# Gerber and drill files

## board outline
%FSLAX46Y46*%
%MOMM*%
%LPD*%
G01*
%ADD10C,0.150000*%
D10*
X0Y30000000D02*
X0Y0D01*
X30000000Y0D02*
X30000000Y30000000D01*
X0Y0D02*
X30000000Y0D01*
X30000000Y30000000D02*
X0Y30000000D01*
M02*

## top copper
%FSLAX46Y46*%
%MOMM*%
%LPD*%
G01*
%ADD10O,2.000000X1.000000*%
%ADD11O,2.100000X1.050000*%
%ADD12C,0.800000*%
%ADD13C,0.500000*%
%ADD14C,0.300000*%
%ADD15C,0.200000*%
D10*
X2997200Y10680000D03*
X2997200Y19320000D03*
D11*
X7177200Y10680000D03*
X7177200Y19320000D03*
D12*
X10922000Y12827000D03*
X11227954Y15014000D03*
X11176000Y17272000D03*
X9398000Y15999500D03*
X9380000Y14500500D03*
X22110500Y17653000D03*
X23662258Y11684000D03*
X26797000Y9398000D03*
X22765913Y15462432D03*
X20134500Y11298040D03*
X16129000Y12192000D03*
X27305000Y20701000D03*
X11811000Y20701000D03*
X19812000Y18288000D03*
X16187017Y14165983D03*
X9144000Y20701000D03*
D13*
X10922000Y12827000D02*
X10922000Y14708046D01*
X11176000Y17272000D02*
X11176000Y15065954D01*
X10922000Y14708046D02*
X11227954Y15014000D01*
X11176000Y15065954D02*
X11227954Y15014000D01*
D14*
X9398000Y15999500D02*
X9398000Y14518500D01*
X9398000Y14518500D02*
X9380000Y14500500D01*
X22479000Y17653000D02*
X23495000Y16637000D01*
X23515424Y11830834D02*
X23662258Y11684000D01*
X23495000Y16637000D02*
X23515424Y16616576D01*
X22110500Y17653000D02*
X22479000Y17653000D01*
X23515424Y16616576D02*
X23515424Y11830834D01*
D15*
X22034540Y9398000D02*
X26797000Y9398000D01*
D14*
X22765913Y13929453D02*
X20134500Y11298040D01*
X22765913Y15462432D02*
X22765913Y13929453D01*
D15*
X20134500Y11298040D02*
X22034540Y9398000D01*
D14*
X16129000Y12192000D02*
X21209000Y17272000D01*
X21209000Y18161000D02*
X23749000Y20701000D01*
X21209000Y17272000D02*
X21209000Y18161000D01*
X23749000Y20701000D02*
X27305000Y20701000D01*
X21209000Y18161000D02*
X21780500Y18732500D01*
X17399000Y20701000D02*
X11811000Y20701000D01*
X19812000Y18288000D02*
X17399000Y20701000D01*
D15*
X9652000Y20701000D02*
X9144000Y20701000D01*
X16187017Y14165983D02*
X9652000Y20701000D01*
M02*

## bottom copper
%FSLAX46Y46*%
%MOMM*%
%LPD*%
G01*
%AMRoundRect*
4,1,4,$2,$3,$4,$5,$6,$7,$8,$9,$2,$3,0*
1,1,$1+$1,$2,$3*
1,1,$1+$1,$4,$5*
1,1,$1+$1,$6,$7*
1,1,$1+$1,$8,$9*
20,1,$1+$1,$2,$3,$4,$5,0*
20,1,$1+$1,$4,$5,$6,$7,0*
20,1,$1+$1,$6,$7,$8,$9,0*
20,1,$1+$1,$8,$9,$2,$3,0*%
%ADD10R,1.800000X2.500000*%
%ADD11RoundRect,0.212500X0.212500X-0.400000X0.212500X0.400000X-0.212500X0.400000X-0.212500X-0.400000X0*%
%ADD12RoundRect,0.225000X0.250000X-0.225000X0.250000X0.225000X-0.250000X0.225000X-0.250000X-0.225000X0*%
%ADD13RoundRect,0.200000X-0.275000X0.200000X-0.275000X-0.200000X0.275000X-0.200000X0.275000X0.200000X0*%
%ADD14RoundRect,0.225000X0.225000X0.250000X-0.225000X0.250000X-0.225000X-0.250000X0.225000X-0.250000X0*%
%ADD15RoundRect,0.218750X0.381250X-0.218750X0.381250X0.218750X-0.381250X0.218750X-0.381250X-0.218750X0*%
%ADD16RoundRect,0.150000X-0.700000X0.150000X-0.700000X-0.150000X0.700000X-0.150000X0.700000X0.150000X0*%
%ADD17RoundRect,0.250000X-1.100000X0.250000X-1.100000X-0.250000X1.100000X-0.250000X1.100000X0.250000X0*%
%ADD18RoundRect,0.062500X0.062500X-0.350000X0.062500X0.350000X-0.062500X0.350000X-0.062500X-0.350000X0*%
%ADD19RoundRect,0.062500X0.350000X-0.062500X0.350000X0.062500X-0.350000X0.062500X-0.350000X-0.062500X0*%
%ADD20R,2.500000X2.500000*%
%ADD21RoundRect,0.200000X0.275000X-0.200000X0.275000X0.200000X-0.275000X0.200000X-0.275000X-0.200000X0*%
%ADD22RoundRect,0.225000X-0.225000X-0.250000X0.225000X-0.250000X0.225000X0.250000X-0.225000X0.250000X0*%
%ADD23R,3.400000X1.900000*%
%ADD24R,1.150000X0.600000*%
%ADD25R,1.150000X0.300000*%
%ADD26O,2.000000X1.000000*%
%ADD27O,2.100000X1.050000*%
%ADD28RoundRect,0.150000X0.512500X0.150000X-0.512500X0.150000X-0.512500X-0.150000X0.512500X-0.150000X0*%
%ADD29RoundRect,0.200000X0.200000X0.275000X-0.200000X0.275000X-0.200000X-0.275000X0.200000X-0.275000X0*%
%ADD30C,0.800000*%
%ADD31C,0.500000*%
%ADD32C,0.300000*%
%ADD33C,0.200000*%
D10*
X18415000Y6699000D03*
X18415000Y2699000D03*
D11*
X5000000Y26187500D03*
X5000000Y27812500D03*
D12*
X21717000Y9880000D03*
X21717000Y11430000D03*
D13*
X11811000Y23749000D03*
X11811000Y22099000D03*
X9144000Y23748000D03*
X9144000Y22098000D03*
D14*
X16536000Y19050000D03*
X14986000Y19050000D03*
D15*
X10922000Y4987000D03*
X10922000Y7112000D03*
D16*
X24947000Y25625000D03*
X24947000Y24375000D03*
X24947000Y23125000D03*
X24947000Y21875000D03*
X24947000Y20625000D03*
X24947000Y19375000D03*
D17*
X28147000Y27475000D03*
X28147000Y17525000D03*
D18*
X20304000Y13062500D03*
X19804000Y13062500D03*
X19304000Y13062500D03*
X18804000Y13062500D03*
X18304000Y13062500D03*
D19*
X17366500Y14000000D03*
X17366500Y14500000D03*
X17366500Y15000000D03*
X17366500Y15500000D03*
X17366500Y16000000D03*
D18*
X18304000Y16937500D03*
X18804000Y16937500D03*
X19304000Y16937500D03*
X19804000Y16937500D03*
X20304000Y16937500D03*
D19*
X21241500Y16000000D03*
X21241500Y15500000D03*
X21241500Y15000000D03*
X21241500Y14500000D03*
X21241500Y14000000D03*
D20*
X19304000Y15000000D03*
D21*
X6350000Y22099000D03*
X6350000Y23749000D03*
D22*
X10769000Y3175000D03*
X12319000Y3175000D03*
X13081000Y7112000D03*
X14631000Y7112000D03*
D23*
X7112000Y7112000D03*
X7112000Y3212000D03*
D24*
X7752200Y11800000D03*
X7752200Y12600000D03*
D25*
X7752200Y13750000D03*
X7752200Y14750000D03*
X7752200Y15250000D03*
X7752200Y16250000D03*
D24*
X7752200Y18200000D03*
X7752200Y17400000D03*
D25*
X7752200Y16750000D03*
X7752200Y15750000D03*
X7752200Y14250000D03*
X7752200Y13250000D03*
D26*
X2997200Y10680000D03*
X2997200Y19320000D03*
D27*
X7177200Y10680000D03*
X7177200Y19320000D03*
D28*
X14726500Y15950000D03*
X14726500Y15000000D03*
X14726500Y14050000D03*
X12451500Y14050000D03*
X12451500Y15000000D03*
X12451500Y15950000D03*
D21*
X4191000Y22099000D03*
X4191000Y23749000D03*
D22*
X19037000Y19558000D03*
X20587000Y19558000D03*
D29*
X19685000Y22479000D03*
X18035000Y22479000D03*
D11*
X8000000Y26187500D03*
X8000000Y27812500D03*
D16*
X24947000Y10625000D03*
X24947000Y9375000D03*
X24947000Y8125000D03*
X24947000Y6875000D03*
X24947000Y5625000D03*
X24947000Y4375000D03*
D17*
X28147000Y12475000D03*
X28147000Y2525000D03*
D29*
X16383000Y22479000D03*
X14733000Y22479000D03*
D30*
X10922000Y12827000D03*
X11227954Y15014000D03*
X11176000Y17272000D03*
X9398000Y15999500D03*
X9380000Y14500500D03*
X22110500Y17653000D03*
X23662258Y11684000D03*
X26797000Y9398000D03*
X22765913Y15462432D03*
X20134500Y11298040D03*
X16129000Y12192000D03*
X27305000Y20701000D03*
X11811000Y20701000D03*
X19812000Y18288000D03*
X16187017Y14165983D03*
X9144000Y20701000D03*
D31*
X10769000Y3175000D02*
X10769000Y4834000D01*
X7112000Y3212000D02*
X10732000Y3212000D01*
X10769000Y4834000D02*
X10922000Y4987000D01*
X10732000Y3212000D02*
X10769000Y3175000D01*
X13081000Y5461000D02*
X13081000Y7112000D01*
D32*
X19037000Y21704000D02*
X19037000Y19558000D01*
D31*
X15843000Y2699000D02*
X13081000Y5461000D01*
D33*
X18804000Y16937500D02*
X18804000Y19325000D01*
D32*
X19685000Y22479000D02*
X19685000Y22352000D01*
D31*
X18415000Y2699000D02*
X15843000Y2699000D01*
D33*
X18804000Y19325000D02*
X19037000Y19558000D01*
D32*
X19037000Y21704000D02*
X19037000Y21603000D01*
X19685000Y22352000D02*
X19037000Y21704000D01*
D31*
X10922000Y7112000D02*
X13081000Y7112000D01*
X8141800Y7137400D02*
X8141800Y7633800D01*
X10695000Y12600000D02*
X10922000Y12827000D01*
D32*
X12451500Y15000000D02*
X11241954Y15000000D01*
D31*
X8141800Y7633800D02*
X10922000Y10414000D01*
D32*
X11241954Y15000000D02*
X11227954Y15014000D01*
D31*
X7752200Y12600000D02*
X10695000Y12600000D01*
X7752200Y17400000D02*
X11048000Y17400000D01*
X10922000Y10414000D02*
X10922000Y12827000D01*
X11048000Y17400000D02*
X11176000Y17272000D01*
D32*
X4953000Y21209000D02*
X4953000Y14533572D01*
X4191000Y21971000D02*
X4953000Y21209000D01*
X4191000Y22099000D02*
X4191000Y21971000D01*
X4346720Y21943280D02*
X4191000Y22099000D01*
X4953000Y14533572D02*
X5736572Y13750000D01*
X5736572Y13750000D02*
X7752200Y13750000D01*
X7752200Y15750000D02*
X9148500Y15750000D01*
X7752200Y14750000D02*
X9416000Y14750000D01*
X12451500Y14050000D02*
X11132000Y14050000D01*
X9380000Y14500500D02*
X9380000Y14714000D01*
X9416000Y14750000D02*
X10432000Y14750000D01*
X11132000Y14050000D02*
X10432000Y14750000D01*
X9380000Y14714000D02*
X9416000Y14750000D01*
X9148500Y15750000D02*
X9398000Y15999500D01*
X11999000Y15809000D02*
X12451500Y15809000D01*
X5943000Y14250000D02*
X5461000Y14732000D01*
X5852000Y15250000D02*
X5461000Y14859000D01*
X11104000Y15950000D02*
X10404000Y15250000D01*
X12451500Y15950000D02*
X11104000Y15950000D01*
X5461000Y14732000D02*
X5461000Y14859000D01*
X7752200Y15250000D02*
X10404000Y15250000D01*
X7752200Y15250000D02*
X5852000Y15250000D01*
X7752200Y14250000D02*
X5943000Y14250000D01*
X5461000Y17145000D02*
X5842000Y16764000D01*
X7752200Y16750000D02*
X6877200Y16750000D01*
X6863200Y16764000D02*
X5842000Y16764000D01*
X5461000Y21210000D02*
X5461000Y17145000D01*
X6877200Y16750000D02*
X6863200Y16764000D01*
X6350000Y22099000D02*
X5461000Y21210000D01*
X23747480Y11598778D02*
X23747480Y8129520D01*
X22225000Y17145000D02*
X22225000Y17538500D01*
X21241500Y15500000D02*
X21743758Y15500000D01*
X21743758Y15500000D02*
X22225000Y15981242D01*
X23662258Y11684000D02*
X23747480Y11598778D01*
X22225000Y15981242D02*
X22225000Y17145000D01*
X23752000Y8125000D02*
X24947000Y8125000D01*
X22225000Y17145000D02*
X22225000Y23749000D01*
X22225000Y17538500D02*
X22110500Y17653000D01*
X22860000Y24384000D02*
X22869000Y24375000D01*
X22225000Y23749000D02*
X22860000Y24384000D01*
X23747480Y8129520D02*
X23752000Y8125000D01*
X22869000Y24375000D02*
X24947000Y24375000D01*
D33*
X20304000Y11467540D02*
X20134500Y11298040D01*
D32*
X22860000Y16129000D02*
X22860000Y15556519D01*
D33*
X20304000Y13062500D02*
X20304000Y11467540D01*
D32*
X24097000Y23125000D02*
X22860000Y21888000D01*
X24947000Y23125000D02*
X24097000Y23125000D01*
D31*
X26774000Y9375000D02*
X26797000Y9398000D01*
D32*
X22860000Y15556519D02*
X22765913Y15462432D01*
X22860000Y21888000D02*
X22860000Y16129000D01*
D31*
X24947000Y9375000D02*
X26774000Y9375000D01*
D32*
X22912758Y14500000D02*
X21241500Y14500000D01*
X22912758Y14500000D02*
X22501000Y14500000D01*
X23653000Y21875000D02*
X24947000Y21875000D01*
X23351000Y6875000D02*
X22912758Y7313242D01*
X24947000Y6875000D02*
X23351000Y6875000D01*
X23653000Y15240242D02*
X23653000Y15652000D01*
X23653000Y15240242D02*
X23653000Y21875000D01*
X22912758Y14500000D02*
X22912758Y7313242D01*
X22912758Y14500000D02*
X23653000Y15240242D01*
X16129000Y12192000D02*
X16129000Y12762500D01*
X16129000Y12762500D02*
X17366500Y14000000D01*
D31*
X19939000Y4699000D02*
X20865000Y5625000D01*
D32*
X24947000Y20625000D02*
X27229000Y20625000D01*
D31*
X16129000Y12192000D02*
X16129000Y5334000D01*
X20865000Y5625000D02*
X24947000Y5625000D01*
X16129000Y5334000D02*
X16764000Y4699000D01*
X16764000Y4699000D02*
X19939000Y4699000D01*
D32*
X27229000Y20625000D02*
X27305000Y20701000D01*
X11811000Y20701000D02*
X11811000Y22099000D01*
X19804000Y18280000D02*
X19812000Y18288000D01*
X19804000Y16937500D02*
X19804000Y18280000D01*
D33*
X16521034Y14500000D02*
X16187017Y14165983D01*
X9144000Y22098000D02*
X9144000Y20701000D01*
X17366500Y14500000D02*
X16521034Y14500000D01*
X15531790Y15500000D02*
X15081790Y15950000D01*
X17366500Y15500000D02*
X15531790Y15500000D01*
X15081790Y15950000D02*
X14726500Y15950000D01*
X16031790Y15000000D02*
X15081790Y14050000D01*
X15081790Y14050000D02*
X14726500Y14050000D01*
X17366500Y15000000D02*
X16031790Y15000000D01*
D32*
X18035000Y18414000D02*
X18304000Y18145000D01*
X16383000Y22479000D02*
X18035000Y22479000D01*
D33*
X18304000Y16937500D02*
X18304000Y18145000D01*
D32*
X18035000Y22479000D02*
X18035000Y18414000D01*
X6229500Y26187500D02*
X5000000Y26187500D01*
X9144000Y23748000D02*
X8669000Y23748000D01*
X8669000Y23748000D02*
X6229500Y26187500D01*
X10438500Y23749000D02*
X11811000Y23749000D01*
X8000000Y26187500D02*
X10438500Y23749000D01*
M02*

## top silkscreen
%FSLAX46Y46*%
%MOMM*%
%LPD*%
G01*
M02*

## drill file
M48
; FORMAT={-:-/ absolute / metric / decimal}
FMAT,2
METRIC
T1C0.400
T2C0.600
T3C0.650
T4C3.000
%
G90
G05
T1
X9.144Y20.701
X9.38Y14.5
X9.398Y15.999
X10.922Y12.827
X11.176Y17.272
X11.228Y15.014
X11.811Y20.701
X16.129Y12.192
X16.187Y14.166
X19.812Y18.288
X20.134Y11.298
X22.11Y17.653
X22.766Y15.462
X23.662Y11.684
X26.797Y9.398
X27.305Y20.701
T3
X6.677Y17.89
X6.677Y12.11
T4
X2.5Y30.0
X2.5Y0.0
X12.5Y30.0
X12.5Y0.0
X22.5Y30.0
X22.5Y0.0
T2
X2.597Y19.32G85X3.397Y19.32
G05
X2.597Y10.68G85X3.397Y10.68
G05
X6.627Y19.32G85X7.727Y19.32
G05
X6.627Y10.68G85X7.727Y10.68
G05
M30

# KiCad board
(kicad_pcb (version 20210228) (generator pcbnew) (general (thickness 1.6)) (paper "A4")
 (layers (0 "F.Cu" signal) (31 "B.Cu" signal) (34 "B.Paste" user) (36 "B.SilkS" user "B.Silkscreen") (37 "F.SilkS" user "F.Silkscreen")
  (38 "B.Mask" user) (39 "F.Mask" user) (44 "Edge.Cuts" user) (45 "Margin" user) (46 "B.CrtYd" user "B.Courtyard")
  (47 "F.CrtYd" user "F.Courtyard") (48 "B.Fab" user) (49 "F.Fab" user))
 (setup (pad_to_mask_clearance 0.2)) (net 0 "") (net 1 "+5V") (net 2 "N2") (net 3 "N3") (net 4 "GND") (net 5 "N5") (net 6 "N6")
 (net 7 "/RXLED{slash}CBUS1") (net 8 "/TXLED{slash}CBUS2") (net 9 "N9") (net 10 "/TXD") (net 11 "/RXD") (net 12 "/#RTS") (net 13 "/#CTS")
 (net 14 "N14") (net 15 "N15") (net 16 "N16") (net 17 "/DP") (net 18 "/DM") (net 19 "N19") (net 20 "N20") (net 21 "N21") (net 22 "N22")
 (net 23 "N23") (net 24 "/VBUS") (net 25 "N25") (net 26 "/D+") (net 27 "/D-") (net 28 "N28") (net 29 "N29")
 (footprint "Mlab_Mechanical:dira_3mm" (layer "F.Cu") (at 20.574 0.254)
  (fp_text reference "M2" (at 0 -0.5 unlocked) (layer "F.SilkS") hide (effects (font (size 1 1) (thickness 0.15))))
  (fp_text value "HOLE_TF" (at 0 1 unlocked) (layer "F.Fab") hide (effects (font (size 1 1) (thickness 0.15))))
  (pad "" np_thru_hole circle (at 1.926 -0.254) (size 3 3) (drill 3) (layers *.Mask)))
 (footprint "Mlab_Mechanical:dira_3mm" (layer "F.Cu") (at 3.302 -29.845)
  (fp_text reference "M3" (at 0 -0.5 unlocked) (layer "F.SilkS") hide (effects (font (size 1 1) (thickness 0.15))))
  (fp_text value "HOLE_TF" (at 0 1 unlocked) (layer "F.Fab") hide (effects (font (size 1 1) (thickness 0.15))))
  (pad "" np_thru_hole circle (at -0.802 -0.155) (size 3 3) (drill 3) (layers *.Mask)))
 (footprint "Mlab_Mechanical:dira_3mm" (layer "F.Cu") (at 15.24 -29.972)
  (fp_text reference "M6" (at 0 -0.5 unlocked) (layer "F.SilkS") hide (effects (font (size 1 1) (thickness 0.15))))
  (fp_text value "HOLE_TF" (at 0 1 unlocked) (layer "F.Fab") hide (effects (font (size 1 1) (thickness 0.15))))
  (pad "" np_thru_hole circle (at -2.74 -0.028) (size 3 3) (drill 3) (layers *.Mask)))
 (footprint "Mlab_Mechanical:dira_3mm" (layer "F.Cu") (at 24.384 -29.845)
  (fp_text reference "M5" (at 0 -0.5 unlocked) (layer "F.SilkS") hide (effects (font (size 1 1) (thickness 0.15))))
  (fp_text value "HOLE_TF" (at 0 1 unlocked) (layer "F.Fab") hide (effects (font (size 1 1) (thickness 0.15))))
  (pad "" np_thru_hole circle (at -1.884 -0.155) (size 3 3) (drill 3) (layers *.Mask)))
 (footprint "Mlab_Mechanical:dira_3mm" (layer "F.Cu") (at 11.43 0)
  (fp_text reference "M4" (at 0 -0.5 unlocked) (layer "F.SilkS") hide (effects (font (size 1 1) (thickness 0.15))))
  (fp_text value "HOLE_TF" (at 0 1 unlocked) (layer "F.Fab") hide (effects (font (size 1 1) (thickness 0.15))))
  (pad "" np_thru_hole circle (at 1.07 0) (size 3 3) (drill 3) (layers *.Mask)))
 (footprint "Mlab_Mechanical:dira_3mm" (layer "F.Cu") (at 2.921 -0.127)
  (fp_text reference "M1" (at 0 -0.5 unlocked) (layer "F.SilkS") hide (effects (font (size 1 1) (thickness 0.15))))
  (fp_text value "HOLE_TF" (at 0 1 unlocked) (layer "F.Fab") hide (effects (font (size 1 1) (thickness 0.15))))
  (pad "" np_thru_hole circle (at -0.421 0.127) (size 3 3) (drill 3) (layers *.Mask)))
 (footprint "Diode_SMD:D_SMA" (layer "B.Cu") (at 18.415 -4.699 -90)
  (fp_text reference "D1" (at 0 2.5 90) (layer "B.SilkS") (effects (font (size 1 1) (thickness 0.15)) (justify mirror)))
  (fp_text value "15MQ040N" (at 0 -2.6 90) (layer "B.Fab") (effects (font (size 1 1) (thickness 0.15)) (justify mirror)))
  (pad "1" smd rect locked (at -2 0 270) (size 2.5 1.8) (layers "B.Cu" "B.Paste" "B.Mask") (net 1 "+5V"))
  (pad "2" smd rect locked (at 2 0 270) (size 2.5 1.8) (layers "B.Cu" "B.Paste" "B.Mask") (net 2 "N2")))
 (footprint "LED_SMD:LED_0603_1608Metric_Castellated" (layer "B.Cu") (at 5 -27 90)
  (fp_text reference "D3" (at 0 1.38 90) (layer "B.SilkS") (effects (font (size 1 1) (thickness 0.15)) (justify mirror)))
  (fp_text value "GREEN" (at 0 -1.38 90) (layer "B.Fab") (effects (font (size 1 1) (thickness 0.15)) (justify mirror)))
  (pad "1" smd roundrect locked (at -0.8125 0 90) (size 1.225 0.85) (layers "B.Cu" "B.Paste" "B.Mask") (roundrect_rratio 0.25) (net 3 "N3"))
  (pad "2" smd roundrect locked (at 0.8125 0 90) (size 1.225 0.85) (layers "B.Cu" "B.Paste" "B.Mask") (roundrect_rratio 0.25) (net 1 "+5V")))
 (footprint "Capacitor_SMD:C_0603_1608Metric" (layer "B.Cu") (at 21.717 -10.655 90)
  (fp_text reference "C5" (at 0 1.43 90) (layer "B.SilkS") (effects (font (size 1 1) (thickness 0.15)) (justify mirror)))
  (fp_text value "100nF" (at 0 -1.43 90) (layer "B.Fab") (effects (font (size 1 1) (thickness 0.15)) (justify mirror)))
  (pad "1" smd roundrect locked (at -0.775 0 90) (size 0.9 0.95) (layers "B.Cu" "B.Paste" "B.Mask") (roundrect_rratio 0.25) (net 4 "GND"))
  (pad "2" smd roundrect locked (at 0.775 0 90) (size 0.9 0.95) (layers "B.Cu" "B.Paste" "B.Mask") (roundrect_rratio 0.25) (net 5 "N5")))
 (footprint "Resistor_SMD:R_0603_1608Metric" (layer "B.Cu") (at 11.811 -22.924 -90)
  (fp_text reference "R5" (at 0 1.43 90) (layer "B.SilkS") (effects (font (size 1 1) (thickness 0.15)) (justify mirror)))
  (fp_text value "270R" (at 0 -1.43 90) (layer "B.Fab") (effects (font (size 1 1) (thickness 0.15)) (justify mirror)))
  (pad "1" smd roundrect locked (at -0.825 0 270) (size 0.8 0.95) (layers "B.Cu" "B.Paste" "B.Mask") (roundrect_rratio 0.25) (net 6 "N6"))
  (pad "2" smd roundrect locked (at 0.825 0 270) (size 0.8 0.95) (layers "B.Cu" "B.Paste" "B.Mask") (roundrect_rratio 0.25)
   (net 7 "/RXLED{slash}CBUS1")))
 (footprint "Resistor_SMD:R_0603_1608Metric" (layer "B.Cu") (at 9.144 -22.923 -90)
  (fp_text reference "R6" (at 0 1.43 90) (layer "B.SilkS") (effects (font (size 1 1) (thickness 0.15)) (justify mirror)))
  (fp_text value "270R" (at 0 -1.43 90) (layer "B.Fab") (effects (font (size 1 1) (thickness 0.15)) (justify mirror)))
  (pad "1" smd roundrect locked (at -0.825 0 270) (size 0.8 0.95) (layers "B.Cu" "B.Paste" "B.Mask") (roundrect_rratio 0.25) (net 3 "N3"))
  (pad "2" smd roundrect locked (at 0.825 0 270) (size 0.8 0.95) (layers "B.Cu" "B.Paste" "B.Mask") (roundrect_rratio 0.25)
   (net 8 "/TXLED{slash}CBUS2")))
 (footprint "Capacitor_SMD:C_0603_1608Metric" (layer "B.Cu") (at 15.761 -19.05 180)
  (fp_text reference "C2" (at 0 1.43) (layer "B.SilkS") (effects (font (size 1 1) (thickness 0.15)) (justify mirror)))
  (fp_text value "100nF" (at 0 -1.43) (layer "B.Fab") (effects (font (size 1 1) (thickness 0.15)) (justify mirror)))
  (pad "1" smd roundrect locked (at -0.775 0 180) (size 0.9 0.95) (layers "B.Cu" "B.Paste" "B.Mask") (roundrect_rratio 0.25) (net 5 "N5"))
  (pad "2" smd roundrect locked (at 0.775 0 180) (size 0.9 0.95) (layers "B.Cu" "B.Paste" "B.Mask") (roundrect_rratio 0.25) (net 4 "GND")))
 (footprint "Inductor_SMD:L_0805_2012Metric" (layer "B.Cu") (at 10.922 -6.0495 90)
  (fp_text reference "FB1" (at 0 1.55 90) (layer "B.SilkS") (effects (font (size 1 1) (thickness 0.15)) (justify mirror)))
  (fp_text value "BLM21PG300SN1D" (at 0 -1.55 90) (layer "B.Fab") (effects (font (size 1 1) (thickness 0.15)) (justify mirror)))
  (pad "1" smd roundrect locked (at -1.0625 0 90) (size 0.875 1.2) (layers "B.Cu" "B.Paste" "B.Mask") (roundrect_rratio 0.25) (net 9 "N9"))
  (pad "2" smd roundrect locked (at 1.0625 0 90) (size 0.875 1.2) (layers "B.Cu" "B.Paste" "B.Mask") (roundrect_rratio 0.25) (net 2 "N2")))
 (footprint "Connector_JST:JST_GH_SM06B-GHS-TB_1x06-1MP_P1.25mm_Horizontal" (layer "B.Cu") (at 26.797 -22.5 -90)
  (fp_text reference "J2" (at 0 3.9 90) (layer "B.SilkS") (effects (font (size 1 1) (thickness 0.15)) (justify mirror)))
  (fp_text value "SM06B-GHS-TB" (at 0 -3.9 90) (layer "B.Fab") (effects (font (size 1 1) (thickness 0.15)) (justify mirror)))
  (pad "1" smd roundrect locked (at -3.125 1.85 270) (size 0.6 1.7) (layers "B.Cu" "B.Paste" "B.Mask") (roundrect_rratio 0.25) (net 1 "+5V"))
  (pad "2" smd roundrect locked (at -1.875 1.85 270) (size 0.6 1.7) (layers "B.Cu" "B.Paste" "B.Mask") (roundrect_rratio 0.25)
   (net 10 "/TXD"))
  (pad "3" smd roundrect locked (at -0.625 1.85 270) (size 0.6 1.7) (layers "B.Cu" "B.Paste" "B.Mask") (roundrect_rratio 0.25)
   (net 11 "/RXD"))
  (pad "4" smd roundrect locked (at 0.625 1.85 270) (size 0.6 1.7) (layers "B.Cu" "B.Paste" "B.Mask") (roundrect_rratio 0.25)
   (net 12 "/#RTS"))
  (pad "5" smd roundrect locked (at 1.875 1.85 270) (size 0.6 1.7) (layers "B.Cu" "B.Paste" "B.Mask") (roundrect_rratio 0.25)
   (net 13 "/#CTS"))
  (pad "6" smd roundrect locked (at 3.125 1.85 270) (size 0.6 1.7) (layers "B.Cu" "B.Paste" "B.Mask") (roundrect_rratio 0.25) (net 4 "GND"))
  (pad "MP" smd roundrect locked (at -4.975 -1.35 270) (size 1 2.7) (layers "B.Cu" "B.Paste" "B.Mask") (roundrect_rratio 0.25) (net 4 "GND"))
  (pad "MP" smd roundrect locked (at 4.975 -1.35 270) (size 1 2.7) (layers "B.Cu" "B.Paste" "B.Mask") (roundrect_rratio 0.25) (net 4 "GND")))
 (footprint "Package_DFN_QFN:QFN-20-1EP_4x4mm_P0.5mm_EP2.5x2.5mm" (layer "B.Cu") (at 19.304 -15 90)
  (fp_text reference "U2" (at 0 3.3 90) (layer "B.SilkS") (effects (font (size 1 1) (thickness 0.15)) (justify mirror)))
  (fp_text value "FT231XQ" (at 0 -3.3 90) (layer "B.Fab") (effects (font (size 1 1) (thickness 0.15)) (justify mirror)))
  (pad "" smd roundrect locked (at -0.625 0.625 90) (size 1.01 1.01) (layers "B.Paste") (roundrect_rratio 0.247525))
  (pad "" smd roundrect locked (at 0.625 0.625 90) (size 1.01 1.01) (layers "B.Paste") (roundrect_rratio 0.247525))
  (pad "" smd roundrect locked (at -0.625 -0.625 90) (size 1.01 1.01) (layers "B.Paste") (roundrect_rratio 0.247525))
  (pad "" smd roundrect locked (at 0.625 -0.625 90) (size 1.01 1.01) (layers "B.Paste") (roundrect_rratio 0.247525))
  (pad "1" smd roundrect locked (at -1.9375 1 90) (size 0.825 0.25) (layers "B.Cu" "B.Paste" "B.Mask") (roundrect_rratio 0.25)
   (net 11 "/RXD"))
  (pad "2" smd roundrect locked (at -1.9375 0.5 90) (size 0.825 0.25) (layers "B.Cu" "B.Paste" "B.Mask") (roundrect_rratio 0.25)
   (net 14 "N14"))
  (pad "3" smd roundrect locked (at -1.9375 0 90) (size 0.825 0.25) (layers "B.Cu" "B.Paste" "B.Mask") (roundrect_rratio 0.25) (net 4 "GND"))
  (pad "4" smd roundrect locked (at -1.9375 -0.5 90) (size 0.825 0.25) (layers "B.Cu" "B.Paste" "B.Mask") (roundrect_rratio 0.25)
   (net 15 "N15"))
  (pad "5" smd roundrect locked (at -1.9375 -1 90) (size 0.825 0.25) (layers "B.Cu" "B.Paste" "B.Mask") (roundrect_rratio 0.25)
   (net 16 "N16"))
  (pad "6" smd roundrect locked (at -1 -1.9375 90) (size 0.25 0.825) (layers "B.Cu" "B.Paste" "B.Mask") (roundrect_rratio 0.25)
   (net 13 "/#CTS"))
  (pad "7" smd roundrect locked (at -0.5 -1.9375 90) (size 0.25 0.825) (layers "B.Cu" "B.Paste" "B.Mask") (roundrect_rratio 0.25)
   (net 8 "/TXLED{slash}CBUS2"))
  (pad "8" smd roundrect locked (at 0 -1.9375 90) (size 0.25 0.825) (layers "B.Cu" "B.Paste" "B.Mask") (roundrect_rratio 0.25)
   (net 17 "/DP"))
  (pad "9" smd roundrect locked (at 0.5 -1.9375 90) (size 0.25 0.825) (layers "B.Cu" "B.Paste" "B.Mask") (roundrect_rratio 0.25)
   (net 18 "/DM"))
  (pad "10" smd roundrect locked (at 1 -1.9375 90) (size 0.25 0.825) (layers "B.Cu" "B.Paste" "B.Mask") (roundrect_rratio 0.25) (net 5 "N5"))
  (pad "11" smd roundrect locked (at 1.9375 -1 90) (size 0.825 0.25) (layers "B.Cu" "B.Paste" "B.Mask") (roundrect_rratio 0.25)
   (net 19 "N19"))
  (pad "12" smd roundrect locked (at 1.9375 -0.5 90) (size 0.825 0.25) (layers "B.Cu" "B.Paste" "B.Mask") (roundrect_rratio 0.25)
   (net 2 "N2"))
  (pad "13" smd roundrect locked (at 1.9375 0 90) (size 0.825 0.25) (layers "B.Cu" "B.Paste" "B.Mask") (roundrect_rratio 0.25) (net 4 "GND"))
  (pad "14" smd roundrect locked (at 1.9375 0.5 90) (size 0.825 0.25) (layers "B.Cu" "B.Paste" "B.Mask") (roundrect_rratio 0.25)
   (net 7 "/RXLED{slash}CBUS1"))
  (pad "15" smd roundrect locked (at 1.9375 1 90) (size 0.825 0.25) (layers "B.Cu" "B.Paste" "B.Mask") (roundrect_rratio 0.25)
   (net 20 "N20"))
  (pad "16" smd roundrect locked (at 1 1.9375 90) (size 0.25 0.825) (layers "B.Cu" "B.Paste" "B.Mask") (roundrect_rratio 0.25)
   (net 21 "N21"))
  (pad "17" smd roundrect locked (at 0.5 1.9375 90) (size 0.25 0.825) (layers "B.Cu" "B.Paste" "B.Mask") (roundrect_rratio 0.25)
   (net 10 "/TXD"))
  (pad "18" smd roundrect locked (at 0 1.9375 90) (size 0.25 0.825) (layers "B.Cu" "B.Paste" "B.Mask") (roundrect_rratio 0.25)
   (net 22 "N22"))
  (pad "19" smd roundrect locked (at -0.5 1.9375 90) (size 0.25 0.825) (layers "B.Cu" "B.Paste" "B.Mask") (roundrect_rratio 0.25)
   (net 12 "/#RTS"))
  (pad "20" smd roundrect locked (at -1 1.9375 90) (size 0.25 0.825) (layers "B.Cu" "B.Paste" "B.Mask") (roundrect_rratio 0.25) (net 5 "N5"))
  (pad "21" smd rect locked (at 0 0 90) (size 2.5 2.5) (layers "B.Cu" "B.Mask") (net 4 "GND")))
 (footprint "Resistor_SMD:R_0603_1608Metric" (layer "B.Cu") (at 6.35 -22.924 90)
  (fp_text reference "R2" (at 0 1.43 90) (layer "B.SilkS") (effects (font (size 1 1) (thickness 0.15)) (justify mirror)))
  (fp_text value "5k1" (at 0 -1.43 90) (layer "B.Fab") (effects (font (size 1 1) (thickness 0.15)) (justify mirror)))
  (pad "1" smd roundrect locked (at -0.825 0 90) (size 0.8 0.95) (layers "B.Cu" "B.Paste" "B.Mask") (roundrect_rratio 0.25) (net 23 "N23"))
  (pad "2" smd roundrect locked (at 0.825 0 90) (size 0.8 0.95) (layers "B.Cu" "B.Paste" "B.Mask") (roundrect_rratio 0.25) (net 4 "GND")))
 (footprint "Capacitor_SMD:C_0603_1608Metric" (layer "B.Cu") (at 11.544 -3.175)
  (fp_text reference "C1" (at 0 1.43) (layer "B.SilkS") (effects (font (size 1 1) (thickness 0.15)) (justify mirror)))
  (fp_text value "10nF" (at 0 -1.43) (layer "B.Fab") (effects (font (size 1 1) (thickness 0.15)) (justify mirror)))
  (pad "1" smd roundrect locked (at -0.775 0) (size 0.9 0.95) (layers "B.Cu" "B.Paste" "B.Mask") (roundrect_rratio 0.25) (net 9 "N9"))
  (pad "2" smd roundrect locked (at 0.775 0) (size 0.9 0.95) (layers "B.Cu" "B.Paste" "B.Mask") (roundrect_rratio 0.25) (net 4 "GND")))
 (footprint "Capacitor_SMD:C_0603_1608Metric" (layer "B.Cu") (at 13.856 -7.112)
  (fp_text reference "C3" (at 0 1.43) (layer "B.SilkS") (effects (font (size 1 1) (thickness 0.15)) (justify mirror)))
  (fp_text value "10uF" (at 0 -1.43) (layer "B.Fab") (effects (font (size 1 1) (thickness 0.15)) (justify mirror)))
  (pad "1" smd roundrect locked (at -0.775 0) (size 0.9 0.95) (layers "B.Cu" "B.Paste" "B.Mask") (roundrect_rratio 0.25) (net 2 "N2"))
  (pad "2" smd roundrect locked (at 0.775 0) (size 0.9 0.95) (layers "B.Cu" "B.Paste" "B.Mask") (roundrect_rratio 0.25) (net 4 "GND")))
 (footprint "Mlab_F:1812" (layer "B.Cu") (at 7.112 -5.162 -90)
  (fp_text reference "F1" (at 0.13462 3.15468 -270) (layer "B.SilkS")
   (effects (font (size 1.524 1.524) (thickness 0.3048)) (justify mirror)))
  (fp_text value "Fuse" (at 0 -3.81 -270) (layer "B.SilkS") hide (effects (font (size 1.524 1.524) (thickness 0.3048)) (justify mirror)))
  (pad "1" smd rect locked (at -1.95 0 270) (size 1.9 3.4) (layers "B.Cu" "B.Paste" "B.Mask") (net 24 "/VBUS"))
  (pad "2" smd rect locked (at 1.95 0 270) (size 1.9 3.4) (layers "B.Cu" "B.Paste" "B.Mask") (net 9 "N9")))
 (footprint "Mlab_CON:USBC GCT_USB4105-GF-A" (layer "B.Cu") (at 2.9972 -15 90)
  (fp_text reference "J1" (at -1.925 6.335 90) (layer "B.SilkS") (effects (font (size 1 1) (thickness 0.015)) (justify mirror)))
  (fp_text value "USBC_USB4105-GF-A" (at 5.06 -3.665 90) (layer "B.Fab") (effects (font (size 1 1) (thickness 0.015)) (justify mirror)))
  (pad "A1/B12" smd rect locked (at -3.2 4.755 90) (size 0.6 1.15) (layers "B.Cu" "B.Paste" "B.Mask") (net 4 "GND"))
  (pad "A4/B9" smd rect locked (at -2.4 4.755 90) (size 0.6 1.15) (layers "B.Cu" "B.Paste" "B.Mask") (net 24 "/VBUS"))
  (pad "A5" smd rect locked (at -1.25 4.755 90) (size 0.3 1.15) (layers "B.Cu" "B.Paste" "B.Mask") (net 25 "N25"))
  (pad "A6" smd rect locked (at -0.25 4.755 90) (size 0.3 1.15) (layers "B.Cu" "B.Paste" "B.Mask") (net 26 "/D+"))
  (pad "A7" smd rect locked (at 0.25 4.755 90) (size 0.3 1.15) (layers "B.Cu" "B.Paste" "B.Mask") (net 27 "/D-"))
  (pad "A8" smd rect locked (at 1.25 4.755 90) (size 0.3 1.15) (layers "B.Cu" "B.Paste" "B.Mask") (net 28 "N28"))
  (pad "B1/A12" smd rect locked (at 3.2 4.755 90) (size 0.6 1.15) (layers "B.Cu" "B.Paste" "B.Mask") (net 4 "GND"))
  (pad "B4/A9" smd rect locked (at 2.4 4.755 90) (size 0.6 1.15) (layers "B.Cu" "B.Paste" "B.Mask") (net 24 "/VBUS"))
  (pad "B5" smd rect locked (at 1.75 4.755 90) (size 0.3 1.15) (layers "B.Cu" "B.Paste" "B.Mask") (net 23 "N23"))
  (pad "B6" smd rect locked (at 0.75 4.755 90) (size 0.3 1.15) (layers "B.Cu" "B.Paste" "B.Mask") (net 26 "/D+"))
  (pad "B7" smd rect locked (at -0.75 4.755 90) (size 0.3 1.15) (layers "B.Cu" "B.Paste" "B.Mask") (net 27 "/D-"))
  (pad "B8" smd rect locked (at -1.75 4.755 90) (size 0.3 1.15) (layers "B.Cu" "B.Paste" "B.Mask") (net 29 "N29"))
  (pad "G1" thru_hole oval locked (at -4.32 0 90) (size 1 2) (drill oval 0.6 1.4) (layers *.Cu *.Mask) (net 4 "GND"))
  (pad "G2" thru_hole oval locked (at 4.32 0 90) (size 1 2) (drill oval 0.6 1.4) (layers *.Cu *.Mask) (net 4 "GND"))
  (pad "G3" thru_hole oval locked (at -4.32 4.18 90) (size 1.05 2.1) (drill oval 0.6 1.7) (layers *.Cu *.Mask) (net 4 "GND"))
  (pad "G4" thru_hole oval locked (at 4.32 4.18 90) (size 1.05 2.1) (drill oval 0.6 1.7) (layers *.Cu *.Mask) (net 4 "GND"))
  (pad "None" np_thru_hole circle locked (at 2.89 3.68 90) (size 0.65 0.65) (drill 0.65) (layers *.Cu *.Mask))
  (pad "None" np_thru_hole circle locked (at -2.89 3.68 90) (size 0.65 0.65) (drill 0.65) (layers *.Cu *.Mask)))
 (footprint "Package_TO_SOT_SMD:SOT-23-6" (layer "B.Cu") (at 13.589 -15 180)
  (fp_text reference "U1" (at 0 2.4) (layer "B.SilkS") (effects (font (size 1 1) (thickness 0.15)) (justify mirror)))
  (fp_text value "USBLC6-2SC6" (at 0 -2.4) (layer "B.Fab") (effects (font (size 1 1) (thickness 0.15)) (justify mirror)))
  (pad "1" smd roundrect locked (at -1.1375 0.95 180) (size 1.325 0.6) (layers "B.Cu" "B.Paste" "B.Mask") (roundrect_rratio 0.25)
   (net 18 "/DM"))
  (pad "2" smd roundrect locked (at -1.1375 0 180) (size 1.325 0.6) (layers "B.Cu" "B.Paste" "B.Mask") (roundrect_rratio 0.25) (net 4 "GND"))
  (pad "3" smd roundrect locked (at -1.1375 -0.95 180) (size 1.325 0.6) (layers "B.Cu" "B.Paste" "B.Mask") (roundrect_rratio 0.25)
   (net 17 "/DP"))
  (pad "4" smd roundrect locked (at 1.1375 -0.95 180) (size 1.325 0.6) (layers "B.Cu" "B.Paste" "B.Mask") (roundrect_rratio 0.25)
   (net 26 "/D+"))
  (pad "5" smd roundrect locked (at 1.1375 0 180) (size 1.325 0.6) (layers "B.Cu" "B.Paste" "B.Mask") (roundrect_rratio 0.25)
   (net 24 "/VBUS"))
  (pad "6" smd roundrect locked (at 1.1375 0.95 180) (size 1.325 0.6) (layers "B.Cu" "B.Paste" "B.Mask") (roundrect_rratio 0.25)
   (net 27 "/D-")))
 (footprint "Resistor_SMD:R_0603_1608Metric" (layer "B.Cu") (at 4.191 -22.924 90)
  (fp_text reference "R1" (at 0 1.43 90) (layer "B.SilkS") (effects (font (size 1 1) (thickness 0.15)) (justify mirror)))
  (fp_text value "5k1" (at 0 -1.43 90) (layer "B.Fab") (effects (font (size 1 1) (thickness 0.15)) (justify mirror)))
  (pad "1" smd roundrect locked (at -0.825 0 90) (size 0.8 0.95) (layers "B.Cu" "B.Paste" "B.Mask") (roundrect_rratio 0.25) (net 25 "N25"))
  (pad "2" smd roundrect locked (at 0.825 0 90) (size 0.8 0.95) (layers "B.Cu" "B.Paste" "B.Mask") (roundrect_rratio 0.25) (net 4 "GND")))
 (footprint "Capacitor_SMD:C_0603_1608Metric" (layer "B.Cu") (at 19.812 -19.558)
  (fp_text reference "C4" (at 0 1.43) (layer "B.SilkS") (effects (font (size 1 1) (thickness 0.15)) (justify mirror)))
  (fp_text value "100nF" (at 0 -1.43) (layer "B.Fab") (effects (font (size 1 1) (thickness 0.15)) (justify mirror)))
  (pad "1" smd roundrect locked (at -0.775 0) (size 0.9 0.95) (layers "B.Cu" "B.Paste" "B.Mask") (roundrect_rratio 0.25) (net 2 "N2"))
  (pad "2" smd roundrect locked (at 0.775 0) (size 0.9 0.95) (layers "B.Cu" "B.Paste" "B.Mask") (roundrect_rratio 0.25) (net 4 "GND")))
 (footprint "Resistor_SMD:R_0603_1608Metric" (layer "B.Cu") (at 18.86 -22.479 180)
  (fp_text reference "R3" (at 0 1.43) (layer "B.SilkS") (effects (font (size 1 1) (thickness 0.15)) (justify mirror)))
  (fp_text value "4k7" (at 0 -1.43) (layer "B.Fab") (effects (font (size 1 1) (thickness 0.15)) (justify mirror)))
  (pad "1" smd roundrect locked (at -0.825 0 180) (size 0.8 0.95) (layers "B.Cu" "B.Paste" "B.Mask") (roundrect_rratio 0.25) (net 2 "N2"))
  (pad "2" smd roundrect locked (at 0.825 0 180) (size 0.8 0.95) (layers "B.Cu" "B.Paste" "B.Mask") (roundrect_rratio 0.25) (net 19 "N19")))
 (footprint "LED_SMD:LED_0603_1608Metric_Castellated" (layer "B.Cu") (at 8 -27 90)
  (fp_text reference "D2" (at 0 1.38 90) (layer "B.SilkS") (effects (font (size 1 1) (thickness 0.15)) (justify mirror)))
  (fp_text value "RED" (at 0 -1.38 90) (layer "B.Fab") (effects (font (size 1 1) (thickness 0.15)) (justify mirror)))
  (pad "1" smd roundrect locked (at -0.8125 0 90) (size 1.225 0.85) (layers "B.Cu" "B.Paste" "B.Mask") (roundrect_rratio 0.25) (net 6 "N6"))
  (pad "2" smd roundrect locked (at 0.8125 0 90) (size 1.225 0.85) (layers "B.Cu" "B.Paste" "B.Mask") (roundrect_rratio 0.25) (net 1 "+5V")))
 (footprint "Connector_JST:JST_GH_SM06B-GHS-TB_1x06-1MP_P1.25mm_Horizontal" (layer "B.Cu") (at 26.797 -7.5 -90)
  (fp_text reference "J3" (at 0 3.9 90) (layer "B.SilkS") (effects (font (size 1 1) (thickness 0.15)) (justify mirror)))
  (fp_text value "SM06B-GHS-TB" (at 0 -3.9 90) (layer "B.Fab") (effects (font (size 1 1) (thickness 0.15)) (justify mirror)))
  (pad "1" smd roundrect locked (at -3.125 1.85 270) (size 0.6 1.7) (layers "B.Cu" "B.Paste" "B.Mask") (roundrect_rratio 0.25) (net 1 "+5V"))
  (pad "2" smd roundrect locked (at -1.875 1.85 270) (size 0.6 1.7) (layers "B.Cu" "B.Paste" "B.Mask") (roundrect_rratio 0.25)
   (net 11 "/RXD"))
  (pad "3" smd roundrect locked (at -0.625 1.85 270) (size 0.6 1.7) (layers "B.Cu" "B.Paste" "B.Mask") (roundrect_rratio 0.25)
   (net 10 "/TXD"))
  (pad "4" smd roundrect locked (at 0.625 1.85 270) (size 0.6 1.7) (layers "B.Cu" "B.Paste" "B.Mask") (roundrect_rratio 0.25)
   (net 12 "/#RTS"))
  (pad "5" smd roundrect locked (at 1.875 1.85 270) (size 0.6 1.7) (layers "B.Cu" "B.Paste" "B.Mask") (roundrect_rratio 0.25)
   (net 13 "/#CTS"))
  (pad "6" smd roundrect locked (at 3.125 1.85 270) (size 0.6 1.7) (layers "B.Cu" "B.Paste" "B.Mask") (roundrect_rratio 0.25) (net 4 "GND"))
  (pad "MP" smd roundrect locked (at -4.975 -1.35 270) (size 1 2.7) (layers "B.Cu" "B.Paste" "B.Mask") (roundrect_rratio 0.25) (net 4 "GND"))
  (pad "MP" smd roundrect locked (at 4.975 -1.35 270) (size 1 2.7) (layers "B.Cu" "B.Paste" "B.Mask") (roundrect_rratio 0.25) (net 4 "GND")))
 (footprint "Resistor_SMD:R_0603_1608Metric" (layer "B.Cu") (at 15.558 -22.479 180)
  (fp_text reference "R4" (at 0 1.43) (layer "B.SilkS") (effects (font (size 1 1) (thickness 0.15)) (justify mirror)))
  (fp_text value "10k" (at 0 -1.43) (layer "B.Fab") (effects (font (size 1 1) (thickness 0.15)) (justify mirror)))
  (pad "1" smd roundrect locked (at -0.825 0 180) (size 0.8 0.95) (layers "B.Cu" "B.Paste" "B.Mask") (roundrect_rratio 0.25) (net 19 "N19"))
  (pad "2" smd roundrect locked (at 0.825 0 180) (size 0.8 0.95) (layers "B.Cu" "B.Paste" "B.Mask") (roundrect_rratio 0.25) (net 4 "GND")))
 (gr_line (start 0 -30) (end 0 0) (layer "Edge.Cuts") (width 0.15))
 (gr_line (start 30 0) (end 30 -30) (layer "Edge.Cuts") (width 0.15))
 (gr_line (start 0 0) (end 30 0) (layer "Edge.Cuts") (width 0.15))
 (gr_line (start 30 -30) (end 0 -30) (layer "Edge.Cuts") (width 0.15))
 (segment (start 10.769 -3.175) (end 10.769 -4.834) (width 0.5) (layer "B.Cu") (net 9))
 (segment (start 7.112 -3.212) (end 10.732 -3.212) (width 0.5) (layer "B.Cu") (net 9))
 (segment (start 10.769 -4.834) (end 10.922 -4.987) (width 0.5) (layer "B.Cu") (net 9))
 (segment (start 10.732 -3.212) (end 10.769 -3.175) (width 0.5) (layer "B.Cu") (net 9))
 (segment (start 13.081 -5.461) (end 13.081 -7.112) (width 0.5) (layer "B.Cu") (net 2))
 (segment (start 19.037 -21.704) (end 19.037 -19.558) (width 0.3) (layer "B.Cu") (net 2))
 (segment (start 15.843 -2.699) (end 13.081 -5.461) (width 0.5) (layer "B.Cu") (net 2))
 (segment (start 18.804 -16.9375) (end 18.804 -19.325) (width 0.2) (layer "B.Cu") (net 2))
 (segment (start 19.685 -22.479) (end 19.685 -22.352) (width 0.3) (layer "B.Cu") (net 2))
 (segment (start 18.415 -2.699) (end 15.843 -2.699) (width 0.5) (layer "B.Cu") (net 2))
 (segment (start 18.804 -19.325) (end 19.037 -19.558) (width 0.2) (layer "B.Cu") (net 2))
 (segment (start 19.037 -21.704) (end 19.037 -21.603) (width 0.3) (layer "B.Cu") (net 2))
 (segment (start 19.685 -22.352) (end 19.037 -21.704) (width 0.3) (layer "B.Cu") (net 2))
 (segment (start 10.922 -7.112) (end 13.081 -7.112) (width 0.5) (layer "B.Cu") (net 2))
 (segment (start 10.922 -12.827) (end 10.922 -14.708046) (width 0.5) (layer "F.Cu") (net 24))
 (segment (start 11.176 -17.272) (end 11.176 -15.065954) (width 0.5) (layer "F.Cu") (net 24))
 (segment (start 10.922 -14.708046) (end 11.227954 -15.014) (width 0.5) (layer "F.Cu") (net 24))
 (segment (start 11.176 -15.065954) (end 11.227954 -15.014) (width 0.5) (layer "F.Cu") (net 24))
 (via (at 10.922 -12.827) (size 0.8) (drill 0.4) (layers "F.Cu" "B.Cu") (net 24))
 (via (at 11.227954 -15.014) (size 0.8) (drill 0.4) (layers "F.Cu" "B.Cu") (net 24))
 (via (at 11.176 -17.272) (size 0.8) (drill 0.4) (layers "F.Cu" "B.Cu") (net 24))
 (segment (start 8.1418 -7.1374) (end 8.1418 -7.6338) (width 0.5) (layer "B.Cu") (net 24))
 (segment (start 10.695 -12.6) (end 10.922 -12.827) (width 0.5) (layer "B.Cu") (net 24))
 (segment (start 12.4515 -15) (end 11.241954 -15) (width 0.3) (layer "B.Cu") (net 24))
 (segment (start 8.1418 -7.6338) (end 10.922 -10.414) (width 0.5) (layer "B.Cu") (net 24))
 (segment (start 11.241954 -15) (end 11.227954 -15.014) (width 0.3) (layer "B.Cu") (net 24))
 (segment (start 7.7522 -12.6) (end 10.695 -12.6) (width 0.5) (layer "B.Cu") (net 24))
 (segment (start 7.7522 -17.4) (end 11.048 -17.4) (width 0.5) (layer "B.Cu") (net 24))
 (segment (start 10.922 -10.414) (end 10.922 -12.827) (width 0.5) (layer "B.Cu") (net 24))
 (segment (start 11.048 -17.4) (end 11.176 -17.272) (width 0.5) (layer "B.Cu") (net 24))
 (segment (start 4.953 -21.209) (end 4.953 -14.533572) (width 0.3) (layer "B.Cu") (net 25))
 (segment (start 4.191 -21.971) (end 4.953 -21.209) (width 0.3) (layer "B.Cu") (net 25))
 (segment (start 4.191 -22.099) (end 4.191 -21.971) (width 0.3) (layer "B.Cu") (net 25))
 (segment (start 4.34672 -21.94328) (end 4.191 -22.099) (width 0.3) (layer "B.Cu") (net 25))
 (segment (start 4.953 -14.533572) (end 5.736572 -13.75) (width 0.3) (layer "B.Cu") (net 25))
 (segment (start 5.736572 -13.75) (end 7.7522 -13.75) (width 0.3) (layer "B.Cu") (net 25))
 (segment (start 9.398 -15.9995) (end 9.398 -14.5185) (width 0.3) (layer "F.Cu") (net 26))
 (segment (start 9.398 -14.5185) (end 9.38 -14.5005) (width 0.3) (layer "F.Cu") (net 26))
 (via (at 9.398 -15.9995) (size 0.8) (drill 0.4) (layers "F.Cu" "B.Cu") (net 26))
 (via (at 9.38 -14.5005) (size 0.8) (drill 0.4) (layers "F.Cu" "B.Cu") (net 26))
 (segment (start 7.7522 -15.75) (end 9.1485 -15.75) (width 0.3) (layer "B.Cu") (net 26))
 (segment (start 7.7522 -14.75) (end 9.416 -14.75) (width 0.3) (layer "B.Cu") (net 26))
 (segment (start 12.4515 -14.05) (end 11.132 -14.05) (width 0.3) (layer "B.Cu") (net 26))
 (segment (start 9.38 -14.5005) (end 9.38 -14.714) (width 0.3) (layer "B.Cu") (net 26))
 (segment (start 9.416 -14.75) (end 10.432 -14.75) (width 0.3) (layer "B.Cu") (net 26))
 (segment (start 11.132 -14.05) (end 10.432 -14.75) (width 0.3) (layer "B.Cu") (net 26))
 (segment (start 9.38 -14.714) (end 9.416 -14.75) (width 0.3) (layer "B.Cu") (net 26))
 (segment (start 9.1485 -15.75) (end 9.398 -15.9995) (width 0.3) (layer "B.Cu") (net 26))
 (segment (start 11.999 -15.809) (end 12.4515 -15.809) (width 0.3) (layer "B.Cu") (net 27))
 (segment (start 5.943 -14.25) (end 5.461 -14.732) (width 0.3) (layer "B.Cu") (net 27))
 (segment (start 5.852 -15.25) (end 5.461 -14.859) (width 0.3) (layer "B.Cu") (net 27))
 (segment (start 11.104 -15.95) (end 10.404 -15.25) (width 0.3) (layer "B.Cu") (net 27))
 (segment (start 12.4515 -15.95) (end 11.104 -15.95) (width 0.3) (layer "B.Cu") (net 27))
 (segment (start 5.461 -14.732) (end 5.461 -14.859) (width 0.3) (layer "B.Cu") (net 27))
 (segment (start 7.7522 -15.25) (end 10.404 -15.25) (width 0.3) (layer "B.Cu") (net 27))
 (segment (start 7.7522 -15.25) (end 5.852 -15.25) (width 0.3) (layer "B.Cu") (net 27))
 (segment (start 7.7522 -14.25) (end 5.943 -14.25) (width 0.3) (layer "B.Cu") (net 27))
 (segment (start 5.461 -17.145) (end 5.842 -16.764) (width 0.3) (layer "B.Cu") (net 23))
 (segment (start 7.7522 -16.75) (end 6.8772 -16.75) (width 0.3) (layer "B.Cu") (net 23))
 (segment (start 6.8632 -16.764) (end 5.842 -16.764) (width 0.3) (layer "B.Cu") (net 23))
 (segment (start 5.461 -21.21) (end 5.461 -17.145) (width 0.3) (layer "B.Cu") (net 23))
 (segment (start 6.8772 -16.75) (end 6.8632 -16.764) (width 0.3) (layer "B.Cu") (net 23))
 (segment (start 6.35 -22.099) (end 5.461 -21.21) (width 0.3) (layer "B.Cu") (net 23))
 (segment (start 22.479 -17.653) (end 23.495 -16.637) (width 0.3) (layer "F.Cu") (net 10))
 (segment (start 23.515424 -11.830834) (end 23.662258 -11.684) (width 0.3) (layer "F.Cu") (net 10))
 (segment (start 23.495 -16.637) (end 23.515424 -16.616576) (width 0.3) (layer "F.Cu") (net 10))
 (segment (start 22.1105 -17.653) (end 22.479 -17.653) (width 0.3) (layer "F.Cu") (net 10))
 (segment (start 23.515424 -16.616576) (end 23.515424 -11.830834) (width 0.3) (layer "F.Cu") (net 10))
 (via (at 22.1105 -17.653) (size 0.8) (drill 0.4) (layers "F.Cu" "B.Cu") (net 10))
 (via (at 23.662258 -11.684) (size 0.8) (drill 0.4) (layers "F.Cu" "B.Cu") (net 10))
 (segment (start 23.74748 -11.598778) (end 23.74748 -8.12952) (width 0.3) (layer "B.Cu") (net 10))
 (segment (start 22.225 -17.145) (end 22.225 -17.5385) (width 0.3) (layer "B.Cu") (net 10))
 (segment (start 21.2415 -15.5) (end 21.743758 -15.5) (width 0.3) (layer "B.Cu") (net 10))
 (segment (start 21.743758 -15.5) (end 22.225 -15.981242) (width 0.3) (layer "B.Cu") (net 10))
 (segment (start 23.662258 -11.684) (end 23.74748 -11.598778) (width 0.3) (layer "B.Cu") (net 10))
 (segment (start 22.225 -15.981242) (end 22.225 -17.145) (width 0.3) (layer "B.Cu") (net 10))
 (segment (start 23.752 -8.125) (end 24.947 -8.125) (width 0.3) (layer "B.Cu") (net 10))
 (segment (start 22.225 -17.145) (end 22.225 -23.749) (width 0.3) (layer "B.Cu") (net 10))
 (segment (start 22.225 -17.5385) (end 22.1105 -17.653) (width 0.3) (layer "B.Cu") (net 10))
 (segment (start 22.86 -24.384) (end 22.869 -24.375) (width 0.3) (layer "B.Cu") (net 10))
 (segment (start 22.225 -23.749) (end 22.86 -24.384) (width 0.3) (layer "B.Cu") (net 10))
 (segment (start 23.74748 -8.12952) (end 23.752 -8.125) (width 0.3) (layer "B.Cu") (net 10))
 (segment (start 22.869 -24.375) (end 24.947 -24.375) (width 0.3) (layer "B.Cu") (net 10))
 (segment (start 22.03454 -9.398) (end 26.797 -9.398) (width 0.2) (layer "F.Cu") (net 11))
 (segment (start 22.765913 -13.929453) (end 20.1345 -11.29804) (width 0.3) (layer "F.Cu") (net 11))
 (segment (start 22.765913 -15.462432) (end 22.765913 -13.929453) (width 0.3) (layer "F.Cu") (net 11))
 (segment (start 20.1345 -11.29804) (end 22.03454 -9.398) (width 0.2) (layer "F.Cu") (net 11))
 (via (at 26.797 -9.398) (size 0.8) (drill 0.4) (layers "F.Cu" "B.Cu") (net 11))
 (via (at 22.765913 -15.462432) (size 0.8) (drill 0.4) (layers "F.Cu" "B.Cu") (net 11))
 (via (at 20.1345 -11.29804) (size 0.8) (drill 0.4) (layers "F.Cu" "B.Cu") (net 11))
 (segment (start 20.304 -11.46754) (end 20.1345 -11.29804) (width 0.2) (layer "B.Cu") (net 11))
 (segment (start 22.86 -16.129) (end 22.86 -15.556519) (width 0.3) (layer "B.Cu") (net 11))
 (segment (start 20.304 -13.0625) (end 20.304 -11.46754) (width 0.2) (layer "B.Cu") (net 11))
 (segment (start 24.097 -23.125) (end 22.86 -21.888) (width 0.3) (layer "B.Cu") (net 11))
 (segment (start 24.947 -23.125) (end 24.097 -23.125) (width 0.3) (layer "B.Cu") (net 11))
 (segment (start 26.774 -9.375) (end 26.797 -9.398) (width 0.5) (layer "B.Cu") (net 11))
 (segment (start 22.86 -15.556519) (end 22.765913 -15.462432) (width 0.3) (layer "B.Cu") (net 11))
 (segment (start 22.86 -21.888) (end 22.86 -16.129) (width 0.3) (layer "B.Cu") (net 11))
 (segment (start 24.947 -9.375) (end 26.774 -9.375) (width 0.5) (layer "B.Cu") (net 11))
 (segment (start 22.912758 -14.5) (end 21.2415 -14.5) (width 0.3) (layer "B.Cu") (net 12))
 (segment (start 22.912758 -14.5) (end 22.501 -14.5) (width 0.3) (layer "B.Cu") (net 12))
 (segment (start 23.653 -21.875) (end 24.947 -21.875) (width 0.3) (layer "B.Cu") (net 12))
 (segment (start 23.351 -6.875) (end 22.912758 -7.313242) (width 0.3) (layer "B.Cu") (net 12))
 (segment (start 24.947 -6.875) (end 23.351 -6.875) (width 0.3) (layer "B.Cu") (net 12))
 (segment (start 23.653 -15.240242) (end 23.653 -15.652) (width 0.3) (layer "B.Cu") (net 12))
 (segment (start 23.653 -15.240242) (end 23.653 -21.875) (width 0.3) (layer "B.Cu") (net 12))
 (segment (start 22.912758 -14.5) (end 22.912758 -7.313242) (width 0.3) (layer "B.Cu") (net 12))
 (segment (start 22.912758 -14.5) (end 23.653 -15.240242) (width 0.3) (layer "B.Cu") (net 12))
 (segment (start 16.129 -12.192) (end 21.209 -17.272) (width 0.3) (layer "F.Cu") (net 13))
 (segment (start 21.209 -18.161) (end 23.749 -20.701) (width 0.3) (layer "F.Cu") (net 13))
 (segment (start 21.209 -17.272) (end 21.209 -18.161) (width 0.3) (layer "F.Cu") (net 13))
 (segment (start 23.749 -20.701) (end 27.305 -20.701) (width 0.3) (layer "F.Cu") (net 13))
 (segment (start 21.209 -18.161) (end 21.7805 -18.7325) (width 0.3) (layer "F.Cu") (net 13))
 (via (at 16.129 -12.192) (size 0.8) (drill 0.4) (layers "F.Cu" "B.Cu") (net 13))
 (via (at 27.305 -20.701) (size 0.8) (drill 0.4) (layers "F.Cu" "B.Cu") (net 13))
 (segment (start 16.129 -12.192) (end 16.129 -12.7625) (width 0.3) (layer "B.Cu") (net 13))
 (segment (start 16.129 -12.7625) (end 17.3665 -14) (width 0.3) (layer "B.Cu") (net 13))
 (segment (start 19.939 -4.699) (end 20.865 -5.625) (width 0.5) (layer "B.Cu") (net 13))
 (segment (start 24.947 -20.625) (end 27.229 -20.625) (width 0.3) (layer "B.Cu") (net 13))
 (segment (start 16.129 -12.192) (end 16.129 -5.334) (width 0.5) (layer "B.Cu") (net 13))
 (segment (start 20.865 -5.625) (end 24.947 -5.625) (width 0.5) (layer "B.Cu") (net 13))
 (segment (start 16.129 -5.334) (end 16.764 -4.699) (width 0.5) (layer "B.Cu") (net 13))
 (segment (start 16.764 -4.699) (end 19.939 -4.699) (width 0.5) (layer "B.Cu") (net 13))
 (segment (start 27.229 -20.625) (end 27.305 -20.701) (width 0.3) (layer "B.Cu") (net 13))
 (segment (start 17.399 -20.701) (end 11.811 -20.701) (width 0.3) (layer "F.Cu") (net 7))
 (segment (start 19.812 -18.288) (end 17.399 -20.701) (width 0.3) (layer "F.Cu") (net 7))
 (via (at 11.811 -20.701) (size 0.8) (drill 0.4) (layers "F.Cu" "B.Cu") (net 7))
 (via (at 19.812 -18.288) (size 0.8) (drill 0.4) (layers "F.Cu" "B.Cu") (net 7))
 (segment (start 11.811 -20.701) (end 11.811 -22.099) (width 0.3) (layer "B.Cu") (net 7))
 (segment (start 19.804 -18.28) (end 19.812 -18.288) (width 0.3) (layer "B.Cu") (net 7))
 (segment (start 19.804 -16.9375) (end 19.804 -18.28) (width 0.3) (layer "B.Cu") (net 7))
 (segment (start 9.652 -20.701) (end 9.144 -20.701) (width 0.2) (layer "F.Cu") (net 8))
 (segment (start 16.187017 -14.165983) (end 9.652 -20.701) (width 0.2) (layer "F.Cu") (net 8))
 (via (at 16.187017 -14.165983) (size 0.8) (drill 0.4) (layers "F.Cu" "B.Cu") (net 8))
 (via (at 9.144 -20.701) (size 0.8) (drill 0.4) (layers "F.Cu" "B.Cu") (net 8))
 (segment (start 16.521034 -14.5) (end 16.187017 -14.165983) (width 0.2) (layer "B.Cu") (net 8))
 (segment (start 9.144 -22.098) (end 9.144 -20.701) (width 0.2) (layer "B.Cu") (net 8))
 (segment (start 17.3665 -14.5) (end 16.521034 -14.5) (width 0.2) (layer "B.Cu") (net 8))
 (segment (start 15.53179 -15.5) (end 15.08179 -15.95) (width 0.2) (layer "B.Cu") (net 18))
 (segment (start 17.3665 -15.5) (end 15.53179 -15.5) (width 0.2) (layer "B.Cu") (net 18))
 (segment (start 15.08179 -15.95) (end 14.7265 -15.95) (width 0.2) (layer "B.Cu") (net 18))
 (segment (start 16.03179 -15) (end 15.08179 -14.05) (width 0.2) (layer "B.Cu") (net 17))
 (segment (start 15.08179 -14.05) (end 14.7265 -14.05) (width 0.2) (layer "B.Cu") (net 17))
 (segment (start 17.3665 -15) (end 16.03179 -15) (width 0.2) (layer "B.Cu") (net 17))
 (segment (start 18.035 -18.414) (end 18.304 -18.145) (width 0.3) (layer "B.Cu") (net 19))
 (segment (start 16.383 -22.479) (end 18.035 -22.479) (width 0.3) (layer "B.Cu") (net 19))
 (segment (start 18.304 -16.9375) (end 18.304 -18.145) (width 0.2) (layer "B.Cu") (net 19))
 (segment (start 18.035 -22.479) (end 18.035 -18.414) (width 0.3) (layer "B.Cu") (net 19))
 (segment (start 6.2295 -26.1875) (end 5 -26.1875) (width 0.3) (layer "B.Cu") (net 3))
 (segment (start 9.144 -23.748) (end 8.669 -23.748) (width 0.3) (layer "B.Cu") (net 3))
 (segment (start 8.669 -23.748) (end 6.2295 -26.1875) (width 0.3) (layer "B.Cu") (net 3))
 (segment (start 10.4385 -23.749) (end 11.811 -23.749) (width 0.3) (layer "B.Cu") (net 6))
 (segment (start 8 -26.1875) (end 10.4385 -23.749) (width 0.3) (layer "B.Cu") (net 6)))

